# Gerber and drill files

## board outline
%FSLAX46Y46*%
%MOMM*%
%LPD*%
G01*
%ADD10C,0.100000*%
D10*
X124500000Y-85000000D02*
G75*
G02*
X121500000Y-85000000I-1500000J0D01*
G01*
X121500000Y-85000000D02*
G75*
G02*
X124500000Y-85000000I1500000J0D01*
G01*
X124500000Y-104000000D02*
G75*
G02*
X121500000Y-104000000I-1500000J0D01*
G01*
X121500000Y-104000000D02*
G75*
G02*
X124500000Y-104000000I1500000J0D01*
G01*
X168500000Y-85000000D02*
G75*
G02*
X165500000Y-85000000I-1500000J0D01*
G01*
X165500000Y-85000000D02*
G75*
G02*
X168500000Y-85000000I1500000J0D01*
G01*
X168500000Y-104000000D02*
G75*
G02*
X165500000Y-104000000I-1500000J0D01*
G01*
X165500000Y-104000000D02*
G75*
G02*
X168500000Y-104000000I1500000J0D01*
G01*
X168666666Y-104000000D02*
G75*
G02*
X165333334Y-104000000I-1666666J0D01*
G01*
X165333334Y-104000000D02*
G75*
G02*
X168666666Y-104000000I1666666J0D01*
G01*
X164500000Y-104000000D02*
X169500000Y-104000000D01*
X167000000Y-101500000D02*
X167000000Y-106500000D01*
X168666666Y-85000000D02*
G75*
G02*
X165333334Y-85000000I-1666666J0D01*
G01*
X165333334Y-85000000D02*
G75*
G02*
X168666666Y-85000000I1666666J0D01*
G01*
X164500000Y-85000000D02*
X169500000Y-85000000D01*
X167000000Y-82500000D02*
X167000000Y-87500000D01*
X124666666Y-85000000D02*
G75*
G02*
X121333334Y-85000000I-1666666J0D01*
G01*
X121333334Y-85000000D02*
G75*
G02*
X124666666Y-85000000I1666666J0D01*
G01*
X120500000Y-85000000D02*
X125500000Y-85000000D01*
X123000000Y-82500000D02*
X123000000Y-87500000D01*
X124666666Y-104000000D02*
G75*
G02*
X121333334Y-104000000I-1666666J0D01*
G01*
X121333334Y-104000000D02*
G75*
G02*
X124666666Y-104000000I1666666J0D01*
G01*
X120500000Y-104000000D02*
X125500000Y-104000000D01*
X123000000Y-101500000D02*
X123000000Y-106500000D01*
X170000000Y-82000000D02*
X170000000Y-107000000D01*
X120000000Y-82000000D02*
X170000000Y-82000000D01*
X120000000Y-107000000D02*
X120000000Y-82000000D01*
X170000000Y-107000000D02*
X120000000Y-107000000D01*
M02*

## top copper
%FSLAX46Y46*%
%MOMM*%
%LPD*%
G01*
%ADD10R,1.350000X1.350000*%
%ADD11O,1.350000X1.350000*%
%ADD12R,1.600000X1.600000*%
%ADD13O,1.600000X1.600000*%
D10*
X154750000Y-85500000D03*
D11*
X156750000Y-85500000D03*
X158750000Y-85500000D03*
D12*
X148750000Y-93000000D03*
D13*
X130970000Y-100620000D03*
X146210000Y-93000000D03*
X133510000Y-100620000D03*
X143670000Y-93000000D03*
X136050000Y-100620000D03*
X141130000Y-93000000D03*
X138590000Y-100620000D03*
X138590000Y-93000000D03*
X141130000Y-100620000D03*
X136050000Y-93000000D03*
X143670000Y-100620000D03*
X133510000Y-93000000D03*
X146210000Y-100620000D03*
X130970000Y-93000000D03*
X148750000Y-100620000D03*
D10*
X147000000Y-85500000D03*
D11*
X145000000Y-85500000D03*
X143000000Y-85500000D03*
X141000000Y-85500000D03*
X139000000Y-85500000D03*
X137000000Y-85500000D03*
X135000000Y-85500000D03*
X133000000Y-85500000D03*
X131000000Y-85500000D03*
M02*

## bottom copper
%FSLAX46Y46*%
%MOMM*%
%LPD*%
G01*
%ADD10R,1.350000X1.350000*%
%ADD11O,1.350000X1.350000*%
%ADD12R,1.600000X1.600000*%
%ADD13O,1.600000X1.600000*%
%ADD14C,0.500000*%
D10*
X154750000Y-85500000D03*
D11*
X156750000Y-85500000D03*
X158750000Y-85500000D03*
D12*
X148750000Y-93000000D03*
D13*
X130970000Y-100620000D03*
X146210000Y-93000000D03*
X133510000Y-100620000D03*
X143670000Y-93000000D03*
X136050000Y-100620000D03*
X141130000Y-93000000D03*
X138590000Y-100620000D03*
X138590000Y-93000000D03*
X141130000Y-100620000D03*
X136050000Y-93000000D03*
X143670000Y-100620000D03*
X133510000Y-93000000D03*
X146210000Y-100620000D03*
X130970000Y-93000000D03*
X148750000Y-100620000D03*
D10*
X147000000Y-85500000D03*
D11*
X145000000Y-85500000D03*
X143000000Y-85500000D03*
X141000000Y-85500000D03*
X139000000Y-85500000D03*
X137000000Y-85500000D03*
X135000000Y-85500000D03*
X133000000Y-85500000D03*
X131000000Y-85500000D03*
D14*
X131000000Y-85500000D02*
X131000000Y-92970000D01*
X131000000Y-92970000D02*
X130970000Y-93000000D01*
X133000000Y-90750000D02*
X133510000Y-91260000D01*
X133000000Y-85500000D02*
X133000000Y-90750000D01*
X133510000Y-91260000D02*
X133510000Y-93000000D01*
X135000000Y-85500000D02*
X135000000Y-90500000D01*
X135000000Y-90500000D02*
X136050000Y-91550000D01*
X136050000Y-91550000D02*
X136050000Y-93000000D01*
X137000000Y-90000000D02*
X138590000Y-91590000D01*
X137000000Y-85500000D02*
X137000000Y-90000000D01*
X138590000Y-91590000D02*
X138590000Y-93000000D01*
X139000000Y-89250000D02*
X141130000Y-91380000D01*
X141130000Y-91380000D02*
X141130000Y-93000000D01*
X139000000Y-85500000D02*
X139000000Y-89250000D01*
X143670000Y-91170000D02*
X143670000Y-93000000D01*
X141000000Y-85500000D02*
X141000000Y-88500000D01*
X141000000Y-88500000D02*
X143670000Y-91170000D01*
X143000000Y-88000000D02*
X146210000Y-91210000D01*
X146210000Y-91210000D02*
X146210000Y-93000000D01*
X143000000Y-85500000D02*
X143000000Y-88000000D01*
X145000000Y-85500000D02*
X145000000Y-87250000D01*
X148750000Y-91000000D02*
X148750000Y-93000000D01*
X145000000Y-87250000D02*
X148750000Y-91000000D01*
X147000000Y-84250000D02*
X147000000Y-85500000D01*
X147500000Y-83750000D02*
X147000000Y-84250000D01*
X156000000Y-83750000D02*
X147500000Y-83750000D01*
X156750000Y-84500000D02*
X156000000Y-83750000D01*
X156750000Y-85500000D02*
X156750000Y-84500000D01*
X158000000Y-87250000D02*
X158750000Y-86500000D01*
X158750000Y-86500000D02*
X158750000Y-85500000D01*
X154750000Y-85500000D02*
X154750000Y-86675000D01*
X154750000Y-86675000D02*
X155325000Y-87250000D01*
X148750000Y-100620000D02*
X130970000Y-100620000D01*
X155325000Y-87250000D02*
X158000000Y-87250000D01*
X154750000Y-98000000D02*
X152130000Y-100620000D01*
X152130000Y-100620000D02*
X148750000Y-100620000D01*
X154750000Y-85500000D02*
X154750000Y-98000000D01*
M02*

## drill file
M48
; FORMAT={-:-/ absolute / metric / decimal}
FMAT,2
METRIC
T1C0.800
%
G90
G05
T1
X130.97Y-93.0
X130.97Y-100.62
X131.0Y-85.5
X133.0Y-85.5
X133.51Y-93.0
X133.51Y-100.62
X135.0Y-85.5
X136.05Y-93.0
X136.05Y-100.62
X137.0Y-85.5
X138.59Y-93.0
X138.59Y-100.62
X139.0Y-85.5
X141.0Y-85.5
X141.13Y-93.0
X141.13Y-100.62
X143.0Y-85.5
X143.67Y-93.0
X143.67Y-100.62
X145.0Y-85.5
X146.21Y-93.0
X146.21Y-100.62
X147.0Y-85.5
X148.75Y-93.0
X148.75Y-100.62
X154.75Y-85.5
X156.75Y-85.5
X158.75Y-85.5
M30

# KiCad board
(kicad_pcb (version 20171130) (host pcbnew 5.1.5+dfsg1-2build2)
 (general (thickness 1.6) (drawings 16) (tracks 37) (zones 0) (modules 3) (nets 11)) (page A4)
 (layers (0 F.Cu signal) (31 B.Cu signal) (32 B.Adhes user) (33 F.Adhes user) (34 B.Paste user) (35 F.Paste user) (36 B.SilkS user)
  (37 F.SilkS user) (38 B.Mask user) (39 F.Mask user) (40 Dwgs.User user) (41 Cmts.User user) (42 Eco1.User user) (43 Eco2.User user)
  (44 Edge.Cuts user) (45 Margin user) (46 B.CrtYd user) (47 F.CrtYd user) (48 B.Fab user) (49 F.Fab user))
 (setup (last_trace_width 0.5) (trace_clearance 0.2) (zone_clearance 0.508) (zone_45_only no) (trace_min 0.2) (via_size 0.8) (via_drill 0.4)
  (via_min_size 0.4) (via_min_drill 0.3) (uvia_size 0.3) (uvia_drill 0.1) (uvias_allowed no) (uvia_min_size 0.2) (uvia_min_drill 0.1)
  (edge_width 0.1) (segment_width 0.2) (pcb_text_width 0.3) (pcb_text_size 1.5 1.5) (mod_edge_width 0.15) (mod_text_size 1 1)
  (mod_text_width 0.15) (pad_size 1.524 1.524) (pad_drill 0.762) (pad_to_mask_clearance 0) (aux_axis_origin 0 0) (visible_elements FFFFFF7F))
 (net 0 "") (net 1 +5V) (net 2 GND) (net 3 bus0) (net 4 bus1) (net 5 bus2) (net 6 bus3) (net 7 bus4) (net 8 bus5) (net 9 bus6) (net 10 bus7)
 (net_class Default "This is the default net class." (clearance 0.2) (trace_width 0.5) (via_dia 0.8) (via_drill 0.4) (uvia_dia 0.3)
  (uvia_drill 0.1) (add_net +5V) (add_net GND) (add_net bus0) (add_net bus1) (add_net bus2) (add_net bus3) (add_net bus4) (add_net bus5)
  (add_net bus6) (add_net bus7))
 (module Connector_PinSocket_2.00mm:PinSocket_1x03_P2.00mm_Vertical (layer F.Cu) (at 154.75 85.5 90)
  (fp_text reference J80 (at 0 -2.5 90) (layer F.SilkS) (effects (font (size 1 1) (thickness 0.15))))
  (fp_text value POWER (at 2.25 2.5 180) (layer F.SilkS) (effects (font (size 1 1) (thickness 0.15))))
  (pad 1 thru_hole rect (at 0 0 90) (size 1.35 1.35) (drill 0.8) (layers *.Cu *.Mask) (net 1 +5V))
  (pad 2 thru_hole oval (at 0 2 90) (size 1.35 1.35) (drill 0.8) (layers *.Cu *.Mask) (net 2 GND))
  (pad 3 thru_hole oval (at 0 4 90) (size 1.35 1.35) (drill 0.8) (layers *.Cu *.Mask) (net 1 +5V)))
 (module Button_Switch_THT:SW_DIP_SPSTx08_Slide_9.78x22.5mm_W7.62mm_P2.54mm (layer F.Cu) (at 148.75 93 270)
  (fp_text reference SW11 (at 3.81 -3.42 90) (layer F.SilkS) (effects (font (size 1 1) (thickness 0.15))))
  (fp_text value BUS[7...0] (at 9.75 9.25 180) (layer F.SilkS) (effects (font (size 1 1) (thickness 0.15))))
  (pad 1 thru_hole rect (at 0 0 270) (size 1.6 1.6) (drill 0.8) (layers *.Cu *.Mask) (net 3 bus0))
  (pad 9 thru_hole oval (at 7.62 17.78 270) (size 1.6 1.6) (drill 0.8) (layers *.Cu *.Mask) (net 1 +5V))
  (pad 2 thru_hole oval (at 0 2.54 270) (size 1.6 1.6) (drill 0.8) (layers *.Cu *.Mask) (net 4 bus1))
  (pad 10 thru_hole oval (at 7.62 15.24 270) (size 1.6 1.6) (drill 0.8) (layers *.Cu *.Mask) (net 1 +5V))
  (pad 3 thru_hole oval (at 0 5.08 270) (size 1.6 1.6) (drill 0.8) (layers *.Cu *.Mask) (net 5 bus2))
  (pad 11 thru_hole oval (at 7.62 12.7 270) (size 1.6 1.6) (drill 0.8) (layers *.Cu *.Mask) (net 1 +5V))
  (pad 4 thru_hole oval (at 0 7.62 270) (size 1.6 1.6) (drill 0.8) (layers *.Cu *.Mask) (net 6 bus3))
  (pad 12 thru_hole oval (at 7.62 10.16 270) (size 1.6 1.6) (drill 0.8) (layers *.Cu *.Mask) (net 1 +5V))
  (pad 5 thru_hole oval (at 0 10.16 270) (size 1.6 1.6) (drill 0.8) (layers *.Cu *.Mask) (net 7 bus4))
  (pad 13 thru_hole oval (at 7.62 7.62 270) (size 1.6 1.6) (drill 0.8) (layers *.Cu *.Mask) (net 1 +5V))
  (pad 6 thru_hole oval (at 0 12.7 270) (size 1.6 1.6) (drill 0.8) (layers *.Cu *.Mask) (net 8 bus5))
  (pad 14 thru_hole oval (at 7.62 5.08 270) (size 1.6 1.6) (drill 0.8) (layers *.Cu *.Mask) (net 1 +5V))
  (pad 7 thru_hole oval (at 0 15.24 270) (size 1.6 1.6) (drill 0.8) (layers *.Cu *.Mask) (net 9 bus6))
  (pad 15 thru_hole oval (at 7.62 2.54 270) (size 1.6 1.6) (drill 0.8) (layers *.Cu *.Mask) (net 1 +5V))
  (pad 8 thru_hole oval (at 0 17.78 270) (size 1.6 1.6) (drill 0.8) (layers *.Cu *.Mask) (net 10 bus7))
  (pad 16 thru_hole oval (at 7.62 0 270) (size 1.6 1.6) (drill 0.8) (layers *.Cu *.Mask) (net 1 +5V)))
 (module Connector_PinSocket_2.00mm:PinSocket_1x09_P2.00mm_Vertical (layer F.Cu) (at 147 85.5 270)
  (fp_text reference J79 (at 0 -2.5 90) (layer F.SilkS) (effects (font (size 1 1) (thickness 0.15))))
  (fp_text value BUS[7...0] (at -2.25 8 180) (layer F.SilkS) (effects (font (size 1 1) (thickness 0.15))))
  (pad 1 thru_hole rect (at 0 0 270) (size 1.35 1.35) (drill 0.8) (layers *.Cu *.Mask) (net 2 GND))
  (pad 2 thru_hole oval (at 0 2 270) (size 1.35 1.35) (drill 0.8) (layers *.Cu *.Mask) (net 3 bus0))
  (pad 3 thru_hole oval (at 0 4 270) (size 1.35 1.35) (drill 0.8) (layers *.Cu *.Mask) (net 4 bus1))
  (pad 4 thru_hole oval (at 0 6 270) (size 1.35 1.35) (drill 0.8) (layers *.Cu *.Mask) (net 5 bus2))
  (pad 5 thru_hole oval (at 0 8 270) (size 1.35 1.35) (drill 0.8) (layers *.Cu *.Mask) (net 6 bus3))
  (pad 6 thru_hole oval (at 0 10 270) (size 1.35 1.35) (drill 0.8) (layers *.Cu *.Mask) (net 7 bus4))
  (pad 7 thru_hole oval (at 0 12 270) (size 1.35 1.35) (drill 0.8) (layers *.Cu *.Mask) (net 8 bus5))
  (pad 8 thru_hole oval (at 0 14 270) (size 1.35 1.35) (drill 0.8) (layers *.Cu *.Mask) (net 9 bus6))
  (pad 9 thru_hole oval (at 0 16 270) (size 1.35 1.35) (drill 0.8) (layers *.Cu *.Mask) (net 10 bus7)))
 (gr_circle (center 123 85) (end 124.5 85) (layer Edge.Cuts) (width 0.1))
 (gr_circle (center 123 104) (end 124.5 104) (layer Edge.Cuts) (width 0.1))
 (gr_circle (center 167 85) (end 168.5 85) (layer Edge.Cuts) (width 0.1))
 (gr_circle (center 167 104) (end 168.5 104) (layer Edge.Cuts) (width 0.1))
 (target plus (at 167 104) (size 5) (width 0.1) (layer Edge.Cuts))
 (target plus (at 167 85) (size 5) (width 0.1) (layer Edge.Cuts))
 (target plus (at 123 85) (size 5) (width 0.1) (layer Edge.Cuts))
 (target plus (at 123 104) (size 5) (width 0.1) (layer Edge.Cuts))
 (gr_line (start 170 82) (end 170 107) (layer Edge.Cuts) (width 0.1))
 (gr_line (start 120 82) (end 170 82) (layer Edge.Cuts) (width 0.1))
 (gr_line (start 120 107) (end 120 82) (layer Edge.Cuts) (width 0.1))
 (gr_line (start 170 107) (end 120 107) (layer Edge.Cuts) (width 0.1))
 (segment (start 131 85.5) (end 131 92.97) (width 0.5) (layer B.Cu) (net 10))
 (segment (start 131 92.97) (end 130.97 93) (width 0.5) (layer B.Cu) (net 10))
 (segment (start 133 90.75) (end 133.51 91.26) (width 0.5) (layer B.Cu) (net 9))
 (segment (start 133 85.5) (end 133 90.75) (width 0.5) (layer B.Cu) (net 9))
 (segment (start 133.51 91.26) (end 133.51 93) (width 0.5) (layer B.Cu) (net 9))
 (segment (start 135 85.5) (end 135 90.5) (width 0.5) (layer B.Cu) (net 8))
 (segment (start 135 90.5) (end 136.05 91.55) (width 0.5) (layer B.Cu) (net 8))
 (segment (start 136.05 91.55) (end 136.05 93) (width 0.5) (layer B.Cu) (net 8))
 (segment (start 137 90) (end 138.59 91.59) (width 0.5) (layer B.Cu) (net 7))
 (segment (start 137 85.5) (end 137 90) (width 0.5) (layer B.Cu) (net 7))
 (segment (start 138.59 91.59) (end 138.59 93) (width 0.5) (layer B.Cu) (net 7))
 (segment (start 139 89.25) (end 141.13 91.38) (width 0.5) (layer B.Cu) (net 6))
 (segment (start 141.13 91.38) (end 141.13 93) (width 0.5) (layer B.Cu) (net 6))
 (segment (start 139 85.5) (end 139 89.25) (width 0.5) (layer B.Cu) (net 6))
 (segment (start 143.67 91.17) (end 143.67 93) (width 0.5) (layer B.Cu) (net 5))
 (segment (start 141 85.5) (end 141 88.5) (width 0.5) (layer B.Cu) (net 5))
 (segment (start 141 88.5) (end 143.67 91.17) (width 0.5) (layer B.Cu) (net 5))
 (segment (start 143 88) (end 146.21 91.21) (width 0.5) (layer B.Cu) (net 4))
 (segment (start 146.21 91.21) (end 146.21 93) (width 0.5) (layer B.Cu) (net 4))
 (segment (start 143 85.5) (end 143 88) (width 0.5) (layer B.Cu) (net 4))
 (segment (start 145 85.5) (end 145 87.25) (width 0.5) (layer B.Cu) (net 3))
 (segment (start 148.75 91) (end 148.75 93) (width 0.5) (layer B.Cu) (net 3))
 (segment (start 145 87.25) (end 148.75 91) (width 0.5) (layer B.Cu) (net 3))
 (segment (start 147 84.25) (end 147 85.5) (width 0.5) (layer B.Cu) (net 2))
 (segment (start 147.5 83.75) (end 147 84.25) (width 0.5) (layer B.Cu) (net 2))
 (segment (start 156 83.75) (end 147.5 83.75) (width 0.5) (layer B.Cu) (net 2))
 (segment (start 156.75 84.5) (end 156 83.75) (width 0.5) (layer B.Cu) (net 2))
 (segment (start 156.75 85.5) (end 156.75 84.5) (width 0.5) (layer B.Cu) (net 2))
 (segment (start 158 87.25) (end 158.75 86.5) (width 0.5) (layer B.Cu) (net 1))
 (segment (start 158.75 86.5) (end 158.75 85.5) (width 0.5) (layer B.Cu) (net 1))
 (segment (start 154.75 85.5) (end 154.75 86.675) (width 0.5) (layer B.Cu) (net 1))
 (segment (start 154.75 86.675) (end 155.325 87.25) (width 0.5) (layer B.Cu) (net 1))
 (segment (start 148.75 100.62) (end 130.97 100.62) (width 0.5) (layer B.Cu) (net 1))
 (segment (start 155.325 87.25) (end 158 87.25) (width 0.5) (layer B.Cu) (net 1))
 (segment (start 154.75 98) (end 152.13 100.62) (width 0.5) (layer B.Cu) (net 1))
 (segment (start 152.13 100.62) (end 148.75 100.62) (width 0.5) (layer B.Cu) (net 1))
 (segment (start 154.75 85.5) (end 154.75 98) (width 0.5) (layer B.Cu) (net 1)))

